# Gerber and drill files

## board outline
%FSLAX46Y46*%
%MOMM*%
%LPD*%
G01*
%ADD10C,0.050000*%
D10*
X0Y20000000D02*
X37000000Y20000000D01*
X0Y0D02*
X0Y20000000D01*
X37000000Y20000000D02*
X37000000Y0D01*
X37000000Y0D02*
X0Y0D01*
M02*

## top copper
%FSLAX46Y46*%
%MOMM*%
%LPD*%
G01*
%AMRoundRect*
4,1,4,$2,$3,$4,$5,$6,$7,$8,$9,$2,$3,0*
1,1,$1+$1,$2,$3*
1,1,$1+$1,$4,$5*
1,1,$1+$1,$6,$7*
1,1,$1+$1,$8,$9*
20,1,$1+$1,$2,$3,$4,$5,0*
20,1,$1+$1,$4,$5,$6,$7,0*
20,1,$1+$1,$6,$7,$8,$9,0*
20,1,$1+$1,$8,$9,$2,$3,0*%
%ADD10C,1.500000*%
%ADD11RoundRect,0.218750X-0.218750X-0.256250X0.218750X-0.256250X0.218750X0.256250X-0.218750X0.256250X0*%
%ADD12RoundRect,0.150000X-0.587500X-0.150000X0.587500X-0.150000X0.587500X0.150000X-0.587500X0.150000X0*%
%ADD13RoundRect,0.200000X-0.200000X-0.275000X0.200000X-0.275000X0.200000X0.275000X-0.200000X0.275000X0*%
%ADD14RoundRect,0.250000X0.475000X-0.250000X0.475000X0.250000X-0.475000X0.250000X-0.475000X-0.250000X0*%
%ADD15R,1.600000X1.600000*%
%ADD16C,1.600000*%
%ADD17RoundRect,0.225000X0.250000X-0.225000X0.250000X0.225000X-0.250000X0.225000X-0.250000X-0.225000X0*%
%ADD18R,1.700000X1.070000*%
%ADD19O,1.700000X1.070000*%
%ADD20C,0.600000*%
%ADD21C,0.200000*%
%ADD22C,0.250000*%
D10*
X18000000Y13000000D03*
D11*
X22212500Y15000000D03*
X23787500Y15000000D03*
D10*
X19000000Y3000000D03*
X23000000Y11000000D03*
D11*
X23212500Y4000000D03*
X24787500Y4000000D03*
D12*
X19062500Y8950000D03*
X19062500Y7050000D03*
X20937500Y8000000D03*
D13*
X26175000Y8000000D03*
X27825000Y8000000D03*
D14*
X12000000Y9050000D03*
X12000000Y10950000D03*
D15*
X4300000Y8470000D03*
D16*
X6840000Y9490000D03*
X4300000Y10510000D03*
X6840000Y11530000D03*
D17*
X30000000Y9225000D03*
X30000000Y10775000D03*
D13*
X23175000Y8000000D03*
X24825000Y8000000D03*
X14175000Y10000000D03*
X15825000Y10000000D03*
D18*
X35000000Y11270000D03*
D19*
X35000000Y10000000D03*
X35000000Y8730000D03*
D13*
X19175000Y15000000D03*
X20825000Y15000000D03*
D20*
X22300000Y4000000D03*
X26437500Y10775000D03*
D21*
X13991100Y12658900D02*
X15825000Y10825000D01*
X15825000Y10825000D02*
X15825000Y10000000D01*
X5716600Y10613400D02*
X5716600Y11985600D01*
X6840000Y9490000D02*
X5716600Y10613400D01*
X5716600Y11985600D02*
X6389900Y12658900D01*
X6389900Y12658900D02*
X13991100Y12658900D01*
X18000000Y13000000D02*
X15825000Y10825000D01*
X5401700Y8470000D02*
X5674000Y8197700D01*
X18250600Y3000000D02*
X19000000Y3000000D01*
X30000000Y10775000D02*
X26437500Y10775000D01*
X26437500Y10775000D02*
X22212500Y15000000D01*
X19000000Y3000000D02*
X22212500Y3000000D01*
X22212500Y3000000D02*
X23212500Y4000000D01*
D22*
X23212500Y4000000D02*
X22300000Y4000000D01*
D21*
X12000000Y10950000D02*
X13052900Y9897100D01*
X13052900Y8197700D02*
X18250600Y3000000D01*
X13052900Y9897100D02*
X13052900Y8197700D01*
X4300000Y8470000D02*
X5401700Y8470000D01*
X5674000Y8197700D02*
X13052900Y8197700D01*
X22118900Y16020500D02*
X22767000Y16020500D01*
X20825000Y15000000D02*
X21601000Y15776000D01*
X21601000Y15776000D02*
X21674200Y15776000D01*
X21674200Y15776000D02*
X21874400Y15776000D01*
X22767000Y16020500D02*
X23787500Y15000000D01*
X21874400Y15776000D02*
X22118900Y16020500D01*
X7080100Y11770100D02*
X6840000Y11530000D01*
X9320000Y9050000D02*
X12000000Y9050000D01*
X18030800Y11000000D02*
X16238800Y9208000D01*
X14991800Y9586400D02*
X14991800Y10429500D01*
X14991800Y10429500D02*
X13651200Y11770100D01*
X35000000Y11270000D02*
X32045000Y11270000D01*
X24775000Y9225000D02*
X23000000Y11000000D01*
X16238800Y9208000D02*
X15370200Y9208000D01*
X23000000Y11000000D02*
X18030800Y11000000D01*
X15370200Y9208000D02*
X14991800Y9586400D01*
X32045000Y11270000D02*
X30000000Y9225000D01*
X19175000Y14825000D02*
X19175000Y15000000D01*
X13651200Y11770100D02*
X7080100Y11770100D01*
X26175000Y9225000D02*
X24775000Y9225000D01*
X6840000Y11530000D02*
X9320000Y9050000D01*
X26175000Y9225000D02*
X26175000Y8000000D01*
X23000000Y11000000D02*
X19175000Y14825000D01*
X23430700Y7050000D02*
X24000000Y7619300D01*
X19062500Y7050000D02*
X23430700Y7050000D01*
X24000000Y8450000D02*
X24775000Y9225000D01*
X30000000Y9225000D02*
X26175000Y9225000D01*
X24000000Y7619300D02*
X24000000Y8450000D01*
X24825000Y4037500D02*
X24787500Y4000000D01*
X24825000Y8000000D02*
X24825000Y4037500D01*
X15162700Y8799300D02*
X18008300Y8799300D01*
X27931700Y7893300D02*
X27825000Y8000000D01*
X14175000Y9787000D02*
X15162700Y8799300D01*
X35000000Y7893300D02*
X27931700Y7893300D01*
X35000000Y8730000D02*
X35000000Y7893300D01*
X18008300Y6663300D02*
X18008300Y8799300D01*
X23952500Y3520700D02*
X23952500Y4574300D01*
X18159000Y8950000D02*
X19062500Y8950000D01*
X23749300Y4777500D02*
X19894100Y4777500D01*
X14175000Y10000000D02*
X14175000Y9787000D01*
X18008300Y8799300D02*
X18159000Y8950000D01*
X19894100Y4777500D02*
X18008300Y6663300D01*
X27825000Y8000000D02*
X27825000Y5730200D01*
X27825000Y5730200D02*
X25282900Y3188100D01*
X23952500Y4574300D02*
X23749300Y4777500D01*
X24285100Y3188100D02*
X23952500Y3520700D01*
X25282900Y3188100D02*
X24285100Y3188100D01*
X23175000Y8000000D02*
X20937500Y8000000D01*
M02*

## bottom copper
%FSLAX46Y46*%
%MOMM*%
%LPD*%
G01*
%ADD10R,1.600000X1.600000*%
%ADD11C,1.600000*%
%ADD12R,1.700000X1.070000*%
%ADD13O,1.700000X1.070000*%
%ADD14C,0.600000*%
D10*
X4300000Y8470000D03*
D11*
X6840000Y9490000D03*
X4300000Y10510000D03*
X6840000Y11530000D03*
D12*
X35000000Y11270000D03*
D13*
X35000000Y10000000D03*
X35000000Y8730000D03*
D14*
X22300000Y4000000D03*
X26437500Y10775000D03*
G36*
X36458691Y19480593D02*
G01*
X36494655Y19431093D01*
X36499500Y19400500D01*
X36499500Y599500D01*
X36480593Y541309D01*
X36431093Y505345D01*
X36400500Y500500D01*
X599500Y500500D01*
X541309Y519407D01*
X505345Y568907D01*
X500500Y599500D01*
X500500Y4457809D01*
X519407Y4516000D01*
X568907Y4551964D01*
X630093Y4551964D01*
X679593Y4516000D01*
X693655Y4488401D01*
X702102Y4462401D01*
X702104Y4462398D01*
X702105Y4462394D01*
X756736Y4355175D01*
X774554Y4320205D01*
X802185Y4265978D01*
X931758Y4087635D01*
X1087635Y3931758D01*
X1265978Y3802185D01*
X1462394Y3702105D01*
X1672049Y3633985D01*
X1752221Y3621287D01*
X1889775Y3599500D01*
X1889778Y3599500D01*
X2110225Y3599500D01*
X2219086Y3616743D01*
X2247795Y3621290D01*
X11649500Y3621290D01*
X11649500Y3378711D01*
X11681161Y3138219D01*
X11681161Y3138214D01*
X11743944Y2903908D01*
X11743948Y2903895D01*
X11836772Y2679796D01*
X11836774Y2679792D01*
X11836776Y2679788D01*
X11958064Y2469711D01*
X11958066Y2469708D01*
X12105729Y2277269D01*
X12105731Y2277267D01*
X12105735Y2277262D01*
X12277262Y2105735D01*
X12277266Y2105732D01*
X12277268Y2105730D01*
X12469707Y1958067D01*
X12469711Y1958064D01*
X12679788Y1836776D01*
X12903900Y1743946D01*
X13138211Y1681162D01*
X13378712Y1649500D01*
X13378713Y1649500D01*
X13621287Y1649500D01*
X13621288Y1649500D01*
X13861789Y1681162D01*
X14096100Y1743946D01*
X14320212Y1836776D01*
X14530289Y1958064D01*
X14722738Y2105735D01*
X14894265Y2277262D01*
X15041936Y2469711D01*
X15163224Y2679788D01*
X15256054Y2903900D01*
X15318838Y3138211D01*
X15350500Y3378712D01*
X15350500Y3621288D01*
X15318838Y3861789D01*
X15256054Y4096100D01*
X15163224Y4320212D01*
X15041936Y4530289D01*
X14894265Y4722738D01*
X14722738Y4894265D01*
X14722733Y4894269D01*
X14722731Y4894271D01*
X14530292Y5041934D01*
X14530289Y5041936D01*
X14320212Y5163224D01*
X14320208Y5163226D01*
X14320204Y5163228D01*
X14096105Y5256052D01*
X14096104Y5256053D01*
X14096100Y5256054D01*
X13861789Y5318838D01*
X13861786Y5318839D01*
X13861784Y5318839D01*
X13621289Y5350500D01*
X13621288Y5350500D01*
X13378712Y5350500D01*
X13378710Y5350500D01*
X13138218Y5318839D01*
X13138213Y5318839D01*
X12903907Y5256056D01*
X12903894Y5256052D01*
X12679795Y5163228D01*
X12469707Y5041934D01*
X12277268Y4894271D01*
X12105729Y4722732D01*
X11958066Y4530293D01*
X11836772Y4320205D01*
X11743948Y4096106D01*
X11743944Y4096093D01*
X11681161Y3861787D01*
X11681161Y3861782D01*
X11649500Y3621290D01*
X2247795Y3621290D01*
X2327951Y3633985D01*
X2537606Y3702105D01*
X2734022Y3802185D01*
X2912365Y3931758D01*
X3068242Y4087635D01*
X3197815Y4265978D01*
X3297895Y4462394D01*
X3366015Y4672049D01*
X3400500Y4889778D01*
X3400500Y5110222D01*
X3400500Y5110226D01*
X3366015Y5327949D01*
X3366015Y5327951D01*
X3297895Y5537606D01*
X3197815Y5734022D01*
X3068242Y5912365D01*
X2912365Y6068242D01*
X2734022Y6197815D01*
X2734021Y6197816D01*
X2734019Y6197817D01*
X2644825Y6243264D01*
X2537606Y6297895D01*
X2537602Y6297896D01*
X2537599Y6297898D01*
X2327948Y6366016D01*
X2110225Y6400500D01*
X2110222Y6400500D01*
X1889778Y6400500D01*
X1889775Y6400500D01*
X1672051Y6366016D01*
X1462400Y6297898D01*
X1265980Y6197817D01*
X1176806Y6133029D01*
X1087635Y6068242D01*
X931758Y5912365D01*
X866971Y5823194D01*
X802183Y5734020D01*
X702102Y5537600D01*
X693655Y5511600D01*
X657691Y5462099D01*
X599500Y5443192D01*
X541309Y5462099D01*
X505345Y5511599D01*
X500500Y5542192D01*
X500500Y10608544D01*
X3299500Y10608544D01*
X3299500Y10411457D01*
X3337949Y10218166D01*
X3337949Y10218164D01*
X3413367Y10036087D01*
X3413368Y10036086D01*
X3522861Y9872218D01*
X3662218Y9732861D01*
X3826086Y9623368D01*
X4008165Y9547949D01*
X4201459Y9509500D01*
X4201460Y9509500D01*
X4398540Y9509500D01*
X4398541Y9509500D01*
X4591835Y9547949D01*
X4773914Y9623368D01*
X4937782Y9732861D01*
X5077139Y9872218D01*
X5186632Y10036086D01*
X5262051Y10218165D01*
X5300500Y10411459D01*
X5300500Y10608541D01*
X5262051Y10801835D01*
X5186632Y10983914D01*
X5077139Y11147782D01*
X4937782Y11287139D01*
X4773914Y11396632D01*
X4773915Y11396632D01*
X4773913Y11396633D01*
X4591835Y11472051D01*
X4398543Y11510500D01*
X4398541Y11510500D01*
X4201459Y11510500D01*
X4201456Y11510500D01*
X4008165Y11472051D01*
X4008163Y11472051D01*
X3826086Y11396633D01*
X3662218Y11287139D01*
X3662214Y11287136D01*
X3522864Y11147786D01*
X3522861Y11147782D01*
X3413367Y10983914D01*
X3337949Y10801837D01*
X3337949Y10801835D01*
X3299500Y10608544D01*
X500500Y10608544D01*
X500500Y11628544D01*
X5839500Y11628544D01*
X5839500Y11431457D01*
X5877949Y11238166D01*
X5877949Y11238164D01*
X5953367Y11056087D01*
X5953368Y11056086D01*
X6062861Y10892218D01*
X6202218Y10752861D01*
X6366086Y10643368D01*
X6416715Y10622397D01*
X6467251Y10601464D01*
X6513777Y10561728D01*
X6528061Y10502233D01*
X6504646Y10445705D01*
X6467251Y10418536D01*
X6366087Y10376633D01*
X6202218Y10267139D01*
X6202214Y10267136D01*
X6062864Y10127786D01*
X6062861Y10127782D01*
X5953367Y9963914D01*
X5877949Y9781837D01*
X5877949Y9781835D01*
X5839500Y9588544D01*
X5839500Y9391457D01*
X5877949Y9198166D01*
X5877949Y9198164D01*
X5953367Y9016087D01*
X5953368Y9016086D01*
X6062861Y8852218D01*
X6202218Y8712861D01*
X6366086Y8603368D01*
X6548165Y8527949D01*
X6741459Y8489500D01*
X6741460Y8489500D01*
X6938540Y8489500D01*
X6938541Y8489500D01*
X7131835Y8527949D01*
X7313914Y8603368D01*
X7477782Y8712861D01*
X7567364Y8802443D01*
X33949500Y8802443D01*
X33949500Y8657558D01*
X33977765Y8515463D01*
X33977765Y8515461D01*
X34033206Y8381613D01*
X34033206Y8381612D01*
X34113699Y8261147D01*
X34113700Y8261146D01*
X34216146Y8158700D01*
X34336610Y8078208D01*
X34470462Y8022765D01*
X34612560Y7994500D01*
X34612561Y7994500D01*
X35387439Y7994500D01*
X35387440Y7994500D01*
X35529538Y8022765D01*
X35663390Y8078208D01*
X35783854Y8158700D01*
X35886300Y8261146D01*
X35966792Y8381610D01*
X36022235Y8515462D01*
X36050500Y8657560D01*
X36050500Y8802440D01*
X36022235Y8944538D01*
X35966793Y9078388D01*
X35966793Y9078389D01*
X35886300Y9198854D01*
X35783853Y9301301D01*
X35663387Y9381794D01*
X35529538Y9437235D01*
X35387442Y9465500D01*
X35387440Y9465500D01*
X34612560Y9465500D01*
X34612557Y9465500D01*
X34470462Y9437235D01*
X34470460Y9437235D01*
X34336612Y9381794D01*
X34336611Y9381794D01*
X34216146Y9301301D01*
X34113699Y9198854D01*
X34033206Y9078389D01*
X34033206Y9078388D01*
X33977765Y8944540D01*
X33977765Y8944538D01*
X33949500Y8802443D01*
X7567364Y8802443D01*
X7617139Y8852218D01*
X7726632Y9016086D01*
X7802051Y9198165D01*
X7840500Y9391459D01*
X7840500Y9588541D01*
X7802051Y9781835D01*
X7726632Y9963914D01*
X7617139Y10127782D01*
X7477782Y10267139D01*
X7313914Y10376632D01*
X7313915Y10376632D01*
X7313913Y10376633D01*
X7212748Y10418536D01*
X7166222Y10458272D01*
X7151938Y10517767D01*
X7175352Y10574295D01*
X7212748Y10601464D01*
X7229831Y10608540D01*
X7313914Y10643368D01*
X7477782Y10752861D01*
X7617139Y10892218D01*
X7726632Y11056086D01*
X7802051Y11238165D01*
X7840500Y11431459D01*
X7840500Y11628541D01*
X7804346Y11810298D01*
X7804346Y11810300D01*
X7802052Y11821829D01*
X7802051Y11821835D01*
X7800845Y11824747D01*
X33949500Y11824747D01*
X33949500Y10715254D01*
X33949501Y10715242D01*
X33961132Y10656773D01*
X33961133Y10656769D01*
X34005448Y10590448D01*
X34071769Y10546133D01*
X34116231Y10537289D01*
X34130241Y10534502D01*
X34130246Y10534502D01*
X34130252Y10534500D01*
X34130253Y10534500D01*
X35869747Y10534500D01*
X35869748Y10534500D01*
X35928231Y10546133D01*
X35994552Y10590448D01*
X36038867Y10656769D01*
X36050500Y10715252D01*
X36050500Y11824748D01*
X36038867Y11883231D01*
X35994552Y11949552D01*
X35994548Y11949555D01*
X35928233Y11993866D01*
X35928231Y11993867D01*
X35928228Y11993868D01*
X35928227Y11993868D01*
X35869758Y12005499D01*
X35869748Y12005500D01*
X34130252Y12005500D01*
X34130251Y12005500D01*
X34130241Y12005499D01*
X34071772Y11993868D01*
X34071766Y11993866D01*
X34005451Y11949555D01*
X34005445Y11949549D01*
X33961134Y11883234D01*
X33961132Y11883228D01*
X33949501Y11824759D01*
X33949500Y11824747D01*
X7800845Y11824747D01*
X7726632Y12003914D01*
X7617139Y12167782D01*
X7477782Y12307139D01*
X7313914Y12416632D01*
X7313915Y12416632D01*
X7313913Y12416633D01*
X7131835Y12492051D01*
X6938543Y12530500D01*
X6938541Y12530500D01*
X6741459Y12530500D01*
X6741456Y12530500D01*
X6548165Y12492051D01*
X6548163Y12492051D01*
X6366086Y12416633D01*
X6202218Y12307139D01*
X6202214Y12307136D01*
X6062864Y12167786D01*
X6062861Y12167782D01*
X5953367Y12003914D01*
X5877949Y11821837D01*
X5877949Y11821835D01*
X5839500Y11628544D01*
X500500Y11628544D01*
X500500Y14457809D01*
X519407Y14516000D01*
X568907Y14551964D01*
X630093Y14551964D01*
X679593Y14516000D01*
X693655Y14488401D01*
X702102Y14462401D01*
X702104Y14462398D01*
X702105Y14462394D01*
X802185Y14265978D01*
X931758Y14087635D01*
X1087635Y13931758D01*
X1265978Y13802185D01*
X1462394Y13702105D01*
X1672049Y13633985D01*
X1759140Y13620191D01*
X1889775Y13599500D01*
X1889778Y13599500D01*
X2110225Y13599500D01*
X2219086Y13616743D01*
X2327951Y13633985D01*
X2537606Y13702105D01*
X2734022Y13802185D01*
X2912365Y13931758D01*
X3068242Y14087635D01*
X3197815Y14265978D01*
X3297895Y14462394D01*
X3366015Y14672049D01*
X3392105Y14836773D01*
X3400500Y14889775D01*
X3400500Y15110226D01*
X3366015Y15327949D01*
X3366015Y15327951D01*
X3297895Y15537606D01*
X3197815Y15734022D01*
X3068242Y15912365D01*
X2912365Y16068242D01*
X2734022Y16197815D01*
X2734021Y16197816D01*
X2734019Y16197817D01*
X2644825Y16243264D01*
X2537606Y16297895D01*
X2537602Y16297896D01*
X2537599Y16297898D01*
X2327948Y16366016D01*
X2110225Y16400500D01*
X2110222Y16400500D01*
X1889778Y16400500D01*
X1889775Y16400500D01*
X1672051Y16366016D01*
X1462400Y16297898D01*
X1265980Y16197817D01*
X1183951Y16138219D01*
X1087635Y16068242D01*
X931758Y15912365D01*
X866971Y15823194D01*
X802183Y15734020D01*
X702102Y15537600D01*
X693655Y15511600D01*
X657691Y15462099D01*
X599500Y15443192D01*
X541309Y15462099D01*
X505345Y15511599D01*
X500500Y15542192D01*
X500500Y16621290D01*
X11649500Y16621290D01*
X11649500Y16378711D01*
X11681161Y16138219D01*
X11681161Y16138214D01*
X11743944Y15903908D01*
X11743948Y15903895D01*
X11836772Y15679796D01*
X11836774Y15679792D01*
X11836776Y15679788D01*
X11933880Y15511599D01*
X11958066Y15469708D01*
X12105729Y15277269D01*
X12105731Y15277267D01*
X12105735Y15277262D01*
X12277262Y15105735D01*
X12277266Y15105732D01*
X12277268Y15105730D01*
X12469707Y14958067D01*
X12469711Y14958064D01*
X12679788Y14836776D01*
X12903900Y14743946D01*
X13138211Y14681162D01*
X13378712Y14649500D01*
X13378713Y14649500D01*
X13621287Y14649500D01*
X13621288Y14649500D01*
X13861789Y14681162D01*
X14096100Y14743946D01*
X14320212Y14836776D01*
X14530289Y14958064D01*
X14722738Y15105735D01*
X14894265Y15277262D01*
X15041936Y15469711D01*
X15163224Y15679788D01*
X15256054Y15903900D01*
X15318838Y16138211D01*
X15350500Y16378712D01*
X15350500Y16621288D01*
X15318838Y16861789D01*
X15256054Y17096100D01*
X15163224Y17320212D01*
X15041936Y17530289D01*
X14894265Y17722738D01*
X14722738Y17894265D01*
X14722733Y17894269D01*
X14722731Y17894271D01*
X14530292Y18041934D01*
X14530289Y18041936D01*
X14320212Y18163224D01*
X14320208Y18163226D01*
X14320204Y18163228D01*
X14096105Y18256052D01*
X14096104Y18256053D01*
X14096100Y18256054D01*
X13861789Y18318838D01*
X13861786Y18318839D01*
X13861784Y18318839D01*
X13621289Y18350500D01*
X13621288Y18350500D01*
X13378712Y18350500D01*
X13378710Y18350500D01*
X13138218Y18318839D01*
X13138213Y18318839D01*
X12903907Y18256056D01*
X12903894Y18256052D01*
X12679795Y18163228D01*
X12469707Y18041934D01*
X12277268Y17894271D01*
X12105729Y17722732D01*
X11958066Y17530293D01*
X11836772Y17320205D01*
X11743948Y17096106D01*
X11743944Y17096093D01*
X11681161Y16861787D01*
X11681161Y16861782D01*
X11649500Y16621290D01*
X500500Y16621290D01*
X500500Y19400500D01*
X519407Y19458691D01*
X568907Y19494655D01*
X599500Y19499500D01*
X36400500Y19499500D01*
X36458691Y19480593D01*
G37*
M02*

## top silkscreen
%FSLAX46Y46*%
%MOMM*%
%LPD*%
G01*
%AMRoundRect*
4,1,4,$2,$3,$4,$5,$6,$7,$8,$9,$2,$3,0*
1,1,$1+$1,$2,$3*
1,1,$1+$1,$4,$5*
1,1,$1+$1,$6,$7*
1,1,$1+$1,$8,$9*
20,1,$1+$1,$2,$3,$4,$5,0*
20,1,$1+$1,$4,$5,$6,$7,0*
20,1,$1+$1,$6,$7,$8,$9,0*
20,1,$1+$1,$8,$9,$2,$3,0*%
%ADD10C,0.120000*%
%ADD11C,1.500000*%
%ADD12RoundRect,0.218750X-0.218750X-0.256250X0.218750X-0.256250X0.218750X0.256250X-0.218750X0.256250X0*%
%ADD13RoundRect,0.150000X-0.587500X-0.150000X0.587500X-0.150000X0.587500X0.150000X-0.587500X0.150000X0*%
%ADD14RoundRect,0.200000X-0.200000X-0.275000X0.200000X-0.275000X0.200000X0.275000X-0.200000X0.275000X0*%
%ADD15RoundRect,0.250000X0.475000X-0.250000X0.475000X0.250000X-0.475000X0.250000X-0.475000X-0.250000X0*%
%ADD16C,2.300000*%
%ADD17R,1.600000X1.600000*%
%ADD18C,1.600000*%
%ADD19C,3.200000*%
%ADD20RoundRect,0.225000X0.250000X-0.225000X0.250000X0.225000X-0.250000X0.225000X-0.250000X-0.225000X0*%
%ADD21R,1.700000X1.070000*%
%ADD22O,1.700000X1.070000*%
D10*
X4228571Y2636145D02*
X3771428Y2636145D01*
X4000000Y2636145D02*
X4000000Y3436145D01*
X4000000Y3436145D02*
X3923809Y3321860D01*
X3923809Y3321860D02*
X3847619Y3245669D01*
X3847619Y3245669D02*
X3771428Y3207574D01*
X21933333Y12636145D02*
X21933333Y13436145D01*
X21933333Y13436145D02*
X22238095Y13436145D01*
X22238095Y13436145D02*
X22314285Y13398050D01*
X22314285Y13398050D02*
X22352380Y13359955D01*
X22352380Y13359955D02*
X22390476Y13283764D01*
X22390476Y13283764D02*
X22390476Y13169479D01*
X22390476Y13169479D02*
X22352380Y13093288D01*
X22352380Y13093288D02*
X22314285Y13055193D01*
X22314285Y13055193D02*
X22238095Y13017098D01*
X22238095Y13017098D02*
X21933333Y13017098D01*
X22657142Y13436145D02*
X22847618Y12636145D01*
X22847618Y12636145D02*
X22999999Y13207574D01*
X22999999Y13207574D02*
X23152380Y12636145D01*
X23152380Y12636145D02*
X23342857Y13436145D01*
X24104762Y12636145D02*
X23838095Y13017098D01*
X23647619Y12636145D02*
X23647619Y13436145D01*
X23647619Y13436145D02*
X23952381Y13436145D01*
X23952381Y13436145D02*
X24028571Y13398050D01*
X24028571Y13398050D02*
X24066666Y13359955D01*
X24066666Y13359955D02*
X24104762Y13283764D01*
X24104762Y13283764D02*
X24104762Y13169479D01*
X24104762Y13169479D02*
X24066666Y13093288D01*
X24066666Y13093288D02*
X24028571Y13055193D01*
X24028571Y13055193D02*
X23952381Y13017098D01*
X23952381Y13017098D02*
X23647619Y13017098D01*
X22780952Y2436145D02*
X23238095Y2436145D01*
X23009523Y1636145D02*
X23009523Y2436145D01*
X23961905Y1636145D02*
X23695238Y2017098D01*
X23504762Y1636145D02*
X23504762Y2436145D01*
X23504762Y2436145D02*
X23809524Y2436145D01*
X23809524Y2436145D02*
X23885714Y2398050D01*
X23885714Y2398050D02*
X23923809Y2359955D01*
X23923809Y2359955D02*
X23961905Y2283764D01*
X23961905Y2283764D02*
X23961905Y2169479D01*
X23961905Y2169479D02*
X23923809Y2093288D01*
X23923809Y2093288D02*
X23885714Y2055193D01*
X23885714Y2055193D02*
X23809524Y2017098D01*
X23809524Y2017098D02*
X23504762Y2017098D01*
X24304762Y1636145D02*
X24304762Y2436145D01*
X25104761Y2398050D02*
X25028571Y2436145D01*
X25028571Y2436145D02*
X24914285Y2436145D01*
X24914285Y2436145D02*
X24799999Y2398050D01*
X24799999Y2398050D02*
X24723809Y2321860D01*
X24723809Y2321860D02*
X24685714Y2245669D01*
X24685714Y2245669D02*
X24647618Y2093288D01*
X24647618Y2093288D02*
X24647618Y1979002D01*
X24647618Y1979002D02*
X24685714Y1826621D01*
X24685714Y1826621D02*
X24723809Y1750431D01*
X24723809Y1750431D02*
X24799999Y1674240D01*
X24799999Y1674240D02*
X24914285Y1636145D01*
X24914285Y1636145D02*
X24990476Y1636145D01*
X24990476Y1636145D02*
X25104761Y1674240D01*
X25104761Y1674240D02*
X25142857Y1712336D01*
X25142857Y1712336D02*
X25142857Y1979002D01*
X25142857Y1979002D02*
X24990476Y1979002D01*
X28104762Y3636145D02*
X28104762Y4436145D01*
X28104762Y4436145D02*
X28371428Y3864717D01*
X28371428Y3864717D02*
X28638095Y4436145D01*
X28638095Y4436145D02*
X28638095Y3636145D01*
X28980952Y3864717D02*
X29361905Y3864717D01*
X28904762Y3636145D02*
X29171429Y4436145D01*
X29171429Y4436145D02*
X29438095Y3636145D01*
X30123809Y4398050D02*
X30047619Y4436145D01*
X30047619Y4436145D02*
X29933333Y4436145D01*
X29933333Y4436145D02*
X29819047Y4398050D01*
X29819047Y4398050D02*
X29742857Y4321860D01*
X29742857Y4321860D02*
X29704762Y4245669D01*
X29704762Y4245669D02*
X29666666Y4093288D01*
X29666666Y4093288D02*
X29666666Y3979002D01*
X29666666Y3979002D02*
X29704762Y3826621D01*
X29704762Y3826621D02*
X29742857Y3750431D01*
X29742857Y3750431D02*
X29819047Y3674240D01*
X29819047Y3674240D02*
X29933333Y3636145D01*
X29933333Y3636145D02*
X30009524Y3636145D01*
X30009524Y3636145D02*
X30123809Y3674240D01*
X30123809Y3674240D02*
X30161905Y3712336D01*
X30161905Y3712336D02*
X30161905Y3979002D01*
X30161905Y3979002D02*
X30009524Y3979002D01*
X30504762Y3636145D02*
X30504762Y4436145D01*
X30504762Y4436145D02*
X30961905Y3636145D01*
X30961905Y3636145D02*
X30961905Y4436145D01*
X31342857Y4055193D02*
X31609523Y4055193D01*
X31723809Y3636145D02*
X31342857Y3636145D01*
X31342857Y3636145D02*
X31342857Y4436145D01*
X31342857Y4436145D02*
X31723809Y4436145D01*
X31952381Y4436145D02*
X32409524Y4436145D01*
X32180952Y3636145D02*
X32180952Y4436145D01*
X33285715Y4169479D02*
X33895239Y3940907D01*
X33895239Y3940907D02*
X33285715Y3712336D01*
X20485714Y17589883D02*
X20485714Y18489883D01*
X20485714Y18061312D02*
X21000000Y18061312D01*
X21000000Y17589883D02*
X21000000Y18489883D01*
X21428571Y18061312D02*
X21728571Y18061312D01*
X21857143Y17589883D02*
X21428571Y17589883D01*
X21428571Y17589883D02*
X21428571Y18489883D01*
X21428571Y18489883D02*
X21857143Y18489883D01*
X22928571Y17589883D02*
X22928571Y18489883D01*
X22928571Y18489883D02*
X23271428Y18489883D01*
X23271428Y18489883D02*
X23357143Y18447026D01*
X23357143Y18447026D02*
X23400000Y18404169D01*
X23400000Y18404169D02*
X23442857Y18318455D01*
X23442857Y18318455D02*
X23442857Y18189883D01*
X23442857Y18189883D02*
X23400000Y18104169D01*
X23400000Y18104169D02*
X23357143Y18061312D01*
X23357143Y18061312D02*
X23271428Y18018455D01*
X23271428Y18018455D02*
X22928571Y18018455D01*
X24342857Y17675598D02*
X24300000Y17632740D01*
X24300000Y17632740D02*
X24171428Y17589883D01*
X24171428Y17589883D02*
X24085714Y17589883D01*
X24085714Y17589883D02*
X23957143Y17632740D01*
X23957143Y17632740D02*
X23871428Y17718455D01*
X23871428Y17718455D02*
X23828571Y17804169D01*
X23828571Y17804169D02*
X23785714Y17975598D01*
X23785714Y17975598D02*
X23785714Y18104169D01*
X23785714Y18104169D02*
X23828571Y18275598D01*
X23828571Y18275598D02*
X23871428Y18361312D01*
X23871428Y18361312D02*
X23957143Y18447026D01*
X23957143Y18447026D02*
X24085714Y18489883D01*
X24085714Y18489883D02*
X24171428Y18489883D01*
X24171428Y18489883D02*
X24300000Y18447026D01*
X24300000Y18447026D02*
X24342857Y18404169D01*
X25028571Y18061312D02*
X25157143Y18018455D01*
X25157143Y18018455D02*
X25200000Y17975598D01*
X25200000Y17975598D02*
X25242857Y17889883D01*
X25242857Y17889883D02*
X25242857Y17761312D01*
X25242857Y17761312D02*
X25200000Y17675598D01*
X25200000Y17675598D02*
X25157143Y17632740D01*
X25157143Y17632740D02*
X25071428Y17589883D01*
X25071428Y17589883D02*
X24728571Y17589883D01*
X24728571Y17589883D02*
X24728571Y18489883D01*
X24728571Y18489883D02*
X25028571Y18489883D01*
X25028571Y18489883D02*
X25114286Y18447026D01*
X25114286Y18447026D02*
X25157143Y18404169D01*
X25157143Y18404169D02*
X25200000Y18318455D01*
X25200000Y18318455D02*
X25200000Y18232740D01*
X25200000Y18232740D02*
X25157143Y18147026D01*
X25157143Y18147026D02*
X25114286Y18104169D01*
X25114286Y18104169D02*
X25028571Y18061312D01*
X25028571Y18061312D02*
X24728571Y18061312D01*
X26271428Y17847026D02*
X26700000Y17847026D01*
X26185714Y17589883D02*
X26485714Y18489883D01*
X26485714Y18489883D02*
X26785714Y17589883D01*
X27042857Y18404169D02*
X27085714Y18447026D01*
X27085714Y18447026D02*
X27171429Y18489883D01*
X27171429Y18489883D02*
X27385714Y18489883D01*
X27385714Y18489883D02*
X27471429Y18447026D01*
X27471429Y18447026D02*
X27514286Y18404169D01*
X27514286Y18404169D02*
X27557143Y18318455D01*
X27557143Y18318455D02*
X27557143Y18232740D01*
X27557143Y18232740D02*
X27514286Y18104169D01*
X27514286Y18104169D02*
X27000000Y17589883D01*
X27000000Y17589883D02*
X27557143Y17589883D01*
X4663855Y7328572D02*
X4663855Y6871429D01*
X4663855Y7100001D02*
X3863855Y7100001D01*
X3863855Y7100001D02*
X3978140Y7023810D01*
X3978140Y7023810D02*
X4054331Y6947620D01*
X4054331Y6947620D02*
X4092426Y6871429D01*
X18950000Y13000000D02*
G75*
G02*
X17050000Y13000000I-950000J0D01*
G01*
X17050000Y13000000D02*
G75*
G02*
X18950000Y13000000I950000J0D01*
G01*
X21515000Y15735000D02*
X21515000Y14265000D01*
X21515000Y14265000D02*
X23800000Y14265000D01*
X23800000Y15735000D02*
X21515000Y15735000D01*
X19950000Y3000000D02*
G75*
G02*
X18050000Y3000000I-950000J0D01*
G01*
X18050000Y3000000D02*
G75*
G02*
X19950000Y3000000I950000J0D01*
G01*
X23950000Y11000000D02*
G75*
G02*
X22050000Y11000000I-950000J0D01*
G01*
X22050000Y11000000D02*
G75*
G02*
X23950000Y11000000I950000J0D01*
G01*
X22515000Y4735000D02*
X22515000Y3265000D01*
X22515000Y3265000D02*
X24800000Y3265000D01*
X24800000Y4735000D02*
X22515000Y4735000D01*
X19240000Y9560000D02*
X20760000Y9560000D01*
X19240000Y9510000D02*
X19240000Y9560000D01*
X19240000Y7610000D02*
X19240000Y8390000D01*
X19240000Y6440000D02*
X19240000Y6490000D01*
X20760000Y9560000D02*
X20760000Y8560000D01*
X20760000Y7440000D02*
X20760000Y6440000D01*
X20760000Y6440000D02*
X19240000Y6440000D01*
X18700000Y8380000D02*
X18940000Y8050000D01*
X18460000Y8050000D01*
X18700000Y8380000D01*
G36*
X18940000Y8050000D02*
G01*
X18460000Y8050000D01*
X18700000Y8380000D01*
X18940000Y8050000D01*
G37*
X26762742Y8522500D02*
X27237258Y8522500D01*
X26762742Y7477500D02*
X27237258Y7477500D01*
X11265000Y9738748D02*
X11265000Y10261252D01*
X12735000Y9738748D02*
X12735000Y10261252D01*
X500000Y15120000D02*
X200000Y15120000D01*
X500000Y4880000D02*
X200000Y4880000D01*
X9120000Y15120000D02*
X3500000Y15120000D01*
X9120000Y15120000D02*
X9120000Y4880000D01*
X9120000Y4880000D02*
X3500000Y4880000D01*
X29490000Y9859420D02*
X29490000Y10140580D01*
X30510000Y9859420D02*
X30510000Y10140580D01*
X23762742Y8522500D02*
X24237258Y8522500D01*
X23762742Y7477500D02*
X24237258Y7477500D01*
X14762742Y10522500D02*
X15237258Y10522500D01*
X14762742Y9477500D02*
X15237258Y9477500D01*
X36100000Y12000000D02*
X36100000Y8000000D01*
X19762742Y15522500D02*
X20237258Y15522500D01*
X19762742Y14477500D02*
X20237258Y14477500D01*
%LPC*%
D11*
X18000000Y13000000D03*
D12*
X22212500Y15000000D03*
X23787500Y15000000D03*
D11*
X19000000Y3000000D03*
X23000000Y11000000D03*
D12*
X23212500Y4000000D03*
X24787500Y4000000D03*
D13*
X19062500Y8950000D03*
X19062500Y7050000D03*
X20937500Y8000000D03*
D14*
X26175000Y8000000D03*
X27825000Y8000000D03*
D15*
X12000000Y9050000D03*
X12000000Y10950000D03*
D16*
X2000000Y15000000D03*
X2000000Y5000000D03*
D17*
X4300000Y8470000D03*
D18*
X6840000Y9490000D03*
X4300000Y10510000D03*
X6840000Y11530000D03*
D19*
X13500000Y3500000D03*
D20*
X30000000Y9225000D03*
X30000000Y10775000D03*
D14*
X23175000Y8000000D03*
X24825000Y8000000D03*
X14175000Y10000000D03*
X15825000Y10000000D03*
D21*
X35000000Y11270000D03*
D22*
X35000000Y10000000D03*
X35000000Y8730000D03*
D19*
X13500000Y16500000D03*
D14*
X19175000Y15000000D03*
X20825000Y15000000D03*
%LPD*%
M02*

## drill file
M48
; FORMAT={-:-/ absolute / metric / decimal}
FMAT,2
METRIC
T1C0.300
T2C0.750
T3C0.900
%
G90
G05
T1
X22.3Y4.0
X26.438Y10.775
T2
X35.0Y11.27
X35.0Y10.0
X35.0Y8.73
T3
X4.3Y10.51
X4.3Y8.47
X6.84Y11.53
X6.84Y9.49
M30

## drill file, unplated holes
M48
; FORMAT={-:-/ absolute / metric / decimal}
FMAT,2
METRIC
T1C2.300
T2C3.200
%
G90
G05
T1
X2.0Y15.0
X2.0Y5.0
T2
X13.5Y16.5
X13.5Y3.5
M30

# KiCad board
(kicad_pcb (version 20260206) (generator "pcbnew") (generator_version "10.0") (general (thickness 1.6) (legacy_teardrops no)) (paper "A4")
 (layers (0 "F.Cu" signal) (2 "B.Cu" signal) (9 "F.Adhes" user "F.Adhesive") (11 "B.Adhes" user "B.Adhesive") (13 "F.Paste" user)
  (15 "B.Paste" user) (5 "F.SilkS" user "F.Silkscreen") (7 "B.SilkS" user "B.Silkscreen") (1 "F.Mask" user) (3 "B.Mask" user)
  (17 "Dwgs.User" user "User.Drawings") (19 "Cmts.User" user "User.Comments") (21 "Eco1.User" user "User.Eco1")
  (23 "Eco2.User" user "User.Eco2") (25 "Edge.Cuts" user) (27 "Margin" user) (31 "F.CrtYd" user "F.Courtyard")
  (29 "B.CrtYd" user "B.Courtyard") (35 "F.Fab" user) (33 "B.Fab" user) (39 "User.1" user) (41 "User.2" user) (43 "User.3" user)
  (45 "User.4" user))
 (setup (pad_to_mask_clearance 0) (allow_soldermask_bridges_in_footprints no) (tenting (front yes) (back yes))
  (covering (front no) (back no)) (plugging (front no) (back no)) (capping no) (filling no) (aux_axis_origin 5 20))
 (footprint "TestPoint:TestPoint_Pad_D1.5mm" (layer "F.Cu") (at 23 7)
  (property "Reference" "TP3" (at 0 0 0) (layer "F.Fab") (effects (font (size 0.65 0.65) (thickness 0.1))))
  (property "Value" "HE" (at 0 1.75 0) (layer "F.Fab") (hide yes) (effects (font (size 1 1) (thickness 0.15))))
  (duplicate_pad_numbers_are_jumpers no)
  (fp_circle (center 0 0) (end 0 0.95) (stroke (width 0.12) (type solid)) (fill no) (layer "F.SilkS"))
  (pad "1" smd circle (at 0 0) (size 1.5 1.5) (layers "F.Cu" "F.Mask") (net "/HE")))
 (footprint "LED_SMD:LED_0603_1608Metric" (layer "F.Cu") (at 28 5)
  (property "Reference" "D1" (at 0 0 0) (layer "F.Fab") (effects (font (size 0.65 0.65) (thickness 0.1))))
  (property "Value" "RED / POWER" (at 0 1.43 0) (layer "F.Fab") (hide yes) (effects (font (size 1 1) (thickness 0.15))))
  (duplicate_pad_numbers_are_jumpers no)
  (fp_line (start -1.485 -0.735) (end -1.485 0.735) (stroke (width 0.12) (type solid)) (layer "F.SilkS"))
  (fp_line (start -1.485 0.735) (end 0.8 0.735) (stroke (width 0.12) (type solid)) (layer "F.SilkS"))
  (fp_line (start 0.8 -0.735) (end -1.485 -0.735) (stroke (width 0.12) (type solid)) (layer "F.SilkS"))
  (pad "1" smd roundrect (at -0.7875 0) (size 0.875 0.95) (layers "F.Cu" "F.Mask" "F.Paste") (roundrect_rratio 0.25) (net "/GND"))
  (pad "2" smd roundrect (at 0.7875 0) (size 0.875 0.95) (layers "F.Cu" "F.Mask" "F.Paste") (roundrect_rratio 0.25) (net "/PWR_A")))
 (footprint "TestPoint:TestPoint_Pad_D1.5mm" (layer "F.Cu") (at 24 17)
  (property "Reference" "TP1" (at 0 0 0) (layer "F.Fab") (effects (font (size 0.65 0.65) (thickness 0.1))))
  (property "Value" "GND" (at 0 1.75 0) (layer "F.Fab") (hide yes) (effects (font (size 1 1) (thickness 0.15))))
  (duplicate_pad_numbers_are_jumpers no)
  (fp_circle (center 0 0) (end 0 0.95) (stroke (width 0.12) (type solid)) (fill no) (layer "F.SilkS"))
  (pad "1" smd circle (at 0 0) (size 1.5 1.5) (layers "F.Cu" "F.Mask") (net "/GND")))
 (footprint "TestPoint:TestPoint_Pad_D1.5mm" (layer "F.Cu") (at 28 9)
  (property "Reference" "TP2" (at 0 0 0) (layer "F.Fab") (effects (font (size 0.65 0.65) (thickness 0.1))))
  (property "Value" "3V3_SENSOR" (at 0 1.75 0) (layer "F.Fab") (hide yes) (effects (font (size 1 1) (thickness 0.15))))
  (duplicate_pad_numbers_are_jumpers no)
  (fp_circle (center 0 0) (end 0 0.95) (stroke (width 0.12) (type solid)) (fill no) (layer "F.SilkS"))
  (pad "1" smd circle (at 0 0) (size 1.5 1.5) (layers "F.Cu" "F.Mask") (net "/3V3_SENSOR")))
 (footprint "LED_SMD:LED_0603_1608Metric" (layer "F.Cu") (at 29 16)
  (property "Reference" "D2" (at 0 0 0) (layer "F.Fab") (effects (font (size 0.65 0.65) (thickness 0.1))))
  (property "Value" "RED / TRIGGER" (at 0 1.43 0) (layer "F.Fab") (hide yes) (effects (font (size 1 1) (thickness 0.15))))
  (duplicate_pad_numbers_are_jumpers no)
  (fp_line (start -1.485 -0.735) (end -1.485 0.735) (stroke (width 0.12) (type solid)) (layer "F.SilkS"))
  (fp_line (start -1.485 0.735) (end 0.8 0.735) (stroke (width 0.12) (type solid)) (layer "F.SilkS"))
  (fp_line (start 0.8 -0.735) (end -1.485 -0.735) (stroke (width 0.12) (type solid)) (layer "F.SilkS"))
  (pad "1" smd roundrect (at -0.7875 0) (size 0.875 0.95) (layers "F.Cu" "F.Mask" "F.Paste") (roundrect_rratio 0.25) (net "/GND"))
  (pad "2" smd roundrect (at 0.7875 0) (size 0.875 0.95) (layers "F.Cu" "F.Mask" "F.Paste") (roundrect_rratio 0.25) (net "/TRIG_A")))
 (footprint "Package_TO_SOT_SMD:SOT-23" (layer "F.Cu") (at 25 12)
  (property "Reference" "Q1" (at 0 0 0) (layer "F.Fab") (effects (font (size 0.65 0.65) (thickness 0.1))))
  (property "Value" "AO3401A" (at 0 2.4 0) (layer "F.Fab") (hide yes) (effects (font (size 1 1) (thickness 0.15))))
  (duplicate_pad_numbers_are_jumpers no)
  (fp_line (start -0.76 -1.56) (end 0.76 -1.56) (stroke (width 0.12) (type solid)) (layer "F.SilkS"))
  (fp_line (start -0.76 -1.51) (end -0.76 -1.56) (stroke (width 0.12) (type solid)) (layer "F.SilkS"))
  (fp_line (start -0.76 0.39) (end -0.76 -0.39) (stroke (width 0.12) (type solid)) (layer "F.SilkS"))
  (fp_line (start -0.76 1.56) (end -0.76 1.51) (stroke (width 0.12) (type solid)) (layer "F.SilkS"))
  (fp_line (start 0.76 -1.56) (end 0.76 -0.56) (stroke (width 0.12) (type solid)) (layer "F.SilkS"))
  (fp_line (start 0.76 0.56) (end 0.76 1.56) (stroke (width 0.12) (type solid)) (layer "F.SilkS"))
  (fp_line (start 0.76 1.56) (end -0.76 1.56) (stroke (width 0.12) (type solid)) (layer "F.SilkS"))
  (fp_poly (pts (xy -1.3 -0.38) (xy -1.06 -0.05) (xy -1.54 -0.05)) (stroke (width 0.12) (type solid)) (fill yes) (layer "F.SilkS"))
  (pad "1" smd roundrect (at -0.9375 -0.95) (size 1.475 0.6) (layers "F.Cu" "F.Mask" "F.Paste") (roundrect_rratio 0.25) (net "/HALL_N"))
  (pad "2" smd roundrect (at -0.9375 0.95) (size 1.475 0.6) (layers "F.Cu" "F.Mask" "F.Paste") (roundrect_rratio 0.25) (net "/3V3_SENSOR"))
  (pad "3" smd roundrect (at 0.9375 0) (size 1.475 0.6) (layers "F.Cu" "F.Mask" "F.Paste") (roundrect_rratio 0.25) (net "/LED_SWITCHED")))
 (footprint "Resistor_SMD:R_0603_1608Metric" (layer "F.Cu") (at 32 12)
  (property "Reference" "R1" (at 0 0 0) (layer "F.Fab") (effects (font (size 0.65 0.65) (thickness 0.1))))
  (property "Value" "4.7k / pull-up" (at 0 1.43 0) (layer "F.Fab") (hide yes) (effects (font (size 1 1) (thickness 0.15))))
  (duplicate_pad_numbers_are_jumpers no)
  (fp_line (start -0.237258 -0.5225) (end 0.237258 -0.5225) (stroke (width 0.12) (type solid)) (layer "F.SilkS"))
  (fp_line (start -0.237258 0.5225) (end 0.237258 0.5225) (stroke (width 0.12) (type solid)) (layer "F.SilkS"))
  (pad "1" smd roundrect (at -0.825 0) (size 0.8 0.95) (layers "F.Cu" "F.Mask" "F.Paste") (roundrect_rratio 0.25) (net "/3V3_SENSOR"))
  (pad "2" smd roundrect (at 0.825 0) (size 0.8 0.95) (layers "F.Cu" "F.Mask" "F.Paste") (roundrect_rratio 0.25) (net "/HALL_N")))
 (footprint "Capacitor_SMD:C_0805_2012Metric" (layer "F.Cu") (at 17 10 90)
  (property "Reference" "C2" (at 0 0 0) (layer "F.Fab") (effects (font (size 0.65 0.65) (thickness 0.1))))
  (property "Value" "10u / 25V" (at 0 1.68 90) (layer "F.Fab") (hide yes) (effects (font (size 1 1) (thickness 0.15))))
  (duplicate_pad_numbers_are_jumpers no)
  (fp_line (start -0.261252 -0.735) (end 0.261252 -0.735) (stroke (width 0.12) (type solid)) (layer "F.SilkS"))
  (fp_line (start -0.261252 0.735) (end 0.261252 0.735) (stroke (width 0.12) (type solid)) (layer "F.SilkS"))
  (pad "1" smd roundrect (at -0.95 0 90) (size 1 1.45) (layers "F.Cu" "F.Mask" "F.Paste") (roundrect_rratio 0.25) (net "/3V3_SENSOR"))
  (pad "2" smd roundrect (at 0.95 0 90) (size 1 1.45) (layers "F.Cu" "F.Mask" "F.Paste") (roundrect_rratio 0.25) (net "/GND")))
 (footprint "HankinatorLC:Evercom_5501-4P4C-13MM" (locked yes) (layer "F.Cu") (at 7 10 -90)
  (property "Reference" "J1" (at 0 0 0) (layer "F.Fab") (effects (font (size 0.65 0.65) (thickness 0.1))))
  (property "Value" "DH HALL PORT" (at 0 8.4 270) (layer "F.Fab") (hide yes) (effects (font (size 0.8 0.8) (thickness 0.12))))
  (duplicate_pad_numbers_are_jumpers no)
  (fp_line (start -5.12 1.5) (end -5.12 1.8) (stroke (width 0.12) (type default)) (layer "F.SilkS"))
  (fp_line (start 5.12 1.5) (end 5.12 1.8) (stroke (width 0.12) (type default)) (layer "F.SilkS"))
  (fp_line (start -5.12 -7.12) (end -5.12 -1.5) (stroke (width 0.12) (type default)) (layer "F.SilkS"))
  (fp_line (start -5.12 -7.12) (end 5.12 -7.12) (stroke (width 0.12) (type default)) (layer "F.SilkS"))
  (fp_line (start 5.12 -7.12) (end 5.12 -1.5) (stroke (width 0.12) (type default)) (layer "F.SilkS"))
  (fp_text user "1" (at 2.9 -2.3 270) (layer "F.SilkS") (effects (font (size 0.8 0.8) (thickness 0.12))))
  (pad "" np_thru_hole circle (at -5 0 270) (size 2.3 2.3) (drill 2.3) (layers "*.Cu" "*.Mask"))
  (pad "" np_thru_hole circle (at 5 0 270) (size 2.3 2.3) (drill 2.3) (layers "*.Cu" "*.Mask"))
  (pad "1" thru_hole rect (at 1.53 -2.3 270) (size 1.6 1.6) (drill 0.9) (layers "*.Cu" "*.Mask") (remove_unused_layers no) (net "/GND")
   (zone_connect 2))
  (pad "2" thru_hole circle (at 0.51 -4.84 270) (size 1.6 1.6) (drill 0.9) (layers "*.Cu" "*.Mask") (remove_unused_layers no) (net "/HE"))
  (pad "3" thru_hole circle (at -0.51 -2.3 270) (size 1.6 1.6) (drill 0.9) (layers "*.Cu" "*.Mask") (remove_unused_layers no)
   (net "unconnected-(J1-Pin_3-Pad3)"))
  (pad "4" thru_hole circle (at -1.53 -4.84 270) (size 1.6 1.6) (drill 0.9) (layers "*.Cu" "*.Mask") (remove_unused_layers no)
   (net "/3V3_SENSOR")))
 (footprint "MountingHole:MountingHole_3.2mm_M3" (layer "F.Cu") (at 18.5 16.5)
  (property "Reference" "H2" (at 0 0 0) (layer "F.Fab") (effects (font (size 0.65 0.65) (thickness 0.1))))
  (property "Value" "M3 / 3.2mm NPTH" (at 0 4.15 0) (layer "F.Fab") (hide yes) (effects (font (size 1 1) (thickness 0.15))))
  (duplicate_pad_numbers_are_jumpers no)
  (pad "" np_thru_hole circle (at 0 0) (size 3.2 3.2) (drill 3.2) (layers "*.Cu" "*.Mask")))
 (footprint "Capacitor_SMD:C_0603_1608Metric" (layer "F.Cu") (at 35 10 90)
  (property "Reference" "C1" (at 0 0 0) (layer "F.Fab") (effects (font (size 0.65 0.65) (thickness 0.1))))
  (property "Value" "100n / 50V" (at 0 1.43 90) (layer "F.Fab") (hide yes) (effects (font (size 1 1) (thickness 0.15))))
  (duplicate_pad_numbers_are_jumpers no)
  (fp_line (start -0.14058 -0.51) (end 0.14058 -0.51) (stroke (width 0.12) (type solid)) (layer "F.SilkS"))
  (fp_line (start -0.14058 0.51) (end 0.14058 0.51) (stroke (width 0.12) (type solid)) (layer "F.SilkS"))
  (pad "1" smd roundrect (at -0.775 0 90) (size 0.9 0.95) (layers "F.Cu" "F.Mask" "F.Paste") (roundrect_rratio 0.25) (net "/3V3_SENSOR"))
  (pad "2" smd roundrect (at 0.775 0 90) (size 0.9 0.95) (layers "F.Cu" "F.Mask" "F.Paste") (roundrect_rratio 0.25) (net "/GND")))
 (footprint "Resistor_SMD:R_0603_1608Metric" (layer "F.Cu") (at 29 12)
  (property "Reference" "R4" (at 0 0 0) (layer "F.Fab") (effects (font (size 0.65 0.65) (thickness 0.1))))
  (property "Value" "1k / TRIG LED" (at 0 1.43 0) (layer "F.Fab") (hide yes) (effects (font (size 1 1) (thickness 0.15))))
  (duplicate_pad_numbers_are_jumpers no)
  (fp_line (start -0.237258 -0.5225) (end 0.237258 -0.5225) (stroke (width 0.12) (type solid)) (layer "F.SilkS"))
  (fp_line (start -0.237258 0.5225) (end 0.237258 0.5225) (stroke (width 0.12) (type solid)) (layer "F.SilkS"))
  (pad "1" smd roundrect (at -0.825 0) (size 0.8 0.95) (layers "F.Cu" "F.Mask" "F.Paste") (roundrect_rratio 0.25) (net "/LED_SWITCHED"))
  (pad "2" smd roundrect (at 0.825 0) (size 0.8 0.95) (layers "F.Cu" "F.Mask" "F.Paste") (roundrect_rratio 0.25) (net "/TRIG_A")))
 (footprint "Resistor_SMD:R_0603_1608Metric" (layer "F.Cu") (at 20 10)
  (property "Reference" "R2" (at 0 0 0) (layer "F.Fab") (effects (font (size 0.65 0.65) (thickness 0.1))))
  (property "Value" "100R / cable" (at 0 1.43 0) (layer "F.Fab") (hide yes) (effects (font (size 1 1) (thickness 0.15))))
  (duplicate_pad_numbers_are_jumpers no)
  (fp_line (start -0.237258 -0.5225) (end 0.237258 -0.5225) (stroke (width 0.12) (type solid)) (layer "F.SilkS"))
  (fp_line (start -0.237258 0.5225) (end 0.237258 0.5225) (stroke (width 0.12) (type solid)) (layer "F.SilkS"))
  (pad "1" smd roundrect (at -0.825 0) (size 0.8 0.95) (layers "F.Cu" "F.Mask" "F.Paste") (roundrect_rratio 0.25) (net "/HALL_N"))
  (pad "2" smd roundrect (at 0.825 0) (size 0.8 0.95) (layers "F.Cu" "F.Mask" "F.Paste") (roundrect_rratio 0.25) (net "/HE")))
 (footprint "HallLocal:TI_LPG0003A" (layer "F.Cu") (at 40 8.73 -90)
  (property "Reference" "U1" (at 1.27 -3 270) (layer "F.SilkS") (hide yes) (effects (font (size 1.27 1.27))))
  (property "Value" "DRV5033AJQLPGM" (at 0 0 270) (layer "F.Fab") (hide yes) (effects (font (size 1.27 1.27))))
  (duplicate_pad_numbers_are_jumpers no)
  (fp_line (start -0.73 -1.1) (end 3.27 -1.1) (stroke (width 0.12) (type default)) (layer "F.SilkS"))
  (pad "1" thru_hole rect (at 0 0 270) (size 1.07 1.7) (drill 0.75) (layers "*.Cu" "*.Mask") (remove_unused_layers no) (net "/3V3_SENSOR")
   (thermal_bridge_angle 45))
  (pad "2" thru_hole oval (at 1.27 0 270) (size 1.07 1.7) (drill 0.75) (layers "*.Cu" "*.Mask") (remove_unused_layers no) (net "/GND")
   (zone_connect 2) (thermal_bridge_angle 45))
  (pad "3" thru_hole oval (at 2.54 0 270) (size 1.07 1.7) (drill 0.75) (layers "*.Cu" "*.Mask") (remove_unused_layers no) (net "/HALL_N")
   (thermal_bridge_angle 45)))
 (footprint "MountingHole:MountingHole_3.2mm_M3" (layer "F.Cu") (at 18.5 3.5)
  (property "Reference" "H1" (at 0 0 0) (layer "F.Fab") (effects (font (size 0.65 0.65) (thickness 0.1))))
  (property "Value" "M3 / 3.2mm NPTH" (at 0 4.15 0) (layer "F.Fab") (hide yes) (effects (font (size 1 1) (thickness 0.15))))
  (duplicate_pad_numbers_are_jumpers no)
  (pad "" np_thru_hole circle (at 0 0) (size 3.2 3.2) (drill 3.2) (layers "*.Cu" "*.Mask")))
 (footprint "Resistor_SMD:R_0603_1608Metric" (layer "F.Cu") (at 25 5)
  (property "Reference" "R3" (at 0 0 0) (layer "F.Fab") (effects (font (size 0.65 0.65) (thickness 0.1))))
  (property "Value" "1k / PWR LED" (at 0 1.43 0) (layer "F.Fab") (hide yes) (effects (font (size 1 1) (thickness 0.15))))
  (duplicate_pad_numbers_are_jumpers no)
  (fp_line (start -0.237258 -0.5225) (end 0.237258 -0.5225) (stroke (width 0.12) (type solid)) (layer "F.SilkS"))
  (fp_line (start -0.237258 0.5225) (end 0.237258 0.5225) (stroke (width 0.12) (type solid)) (layer "F.SilkS"))
  (pad "1" smd roundrect (at -0.825 0) (size 0.8 0.95) (layers "F.Cu" "F.Mask" "F.Paste") (roundrect_rratio 0.25) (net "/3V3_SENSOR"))
  (pad "2" smd roundrect (at 0.825 0) (size 0.8 0.95) (layers "F.Cu" "F.Mask" "F.Paste") (roundrect_rratio 0.25) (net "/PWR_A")))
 (gr_line (start 5 0) (end 42 0) (stroke (width 0.05) (type default)) (layer "Edge.Cuts"))
 (gr_line (start 5 20) (end 5 0) (stroke (width 0.05) (type default)) (layer "Edge.Cuts"))
 (gr_line (start 42 0) (end 42 20) (stroke (width 0.05) (type default)) (layer "Edge.Cuts"))
 (gr_line (start 42 20) (end 5 20) (stroke (width 0.05) (type default)) (layer "Edge.Cuts"))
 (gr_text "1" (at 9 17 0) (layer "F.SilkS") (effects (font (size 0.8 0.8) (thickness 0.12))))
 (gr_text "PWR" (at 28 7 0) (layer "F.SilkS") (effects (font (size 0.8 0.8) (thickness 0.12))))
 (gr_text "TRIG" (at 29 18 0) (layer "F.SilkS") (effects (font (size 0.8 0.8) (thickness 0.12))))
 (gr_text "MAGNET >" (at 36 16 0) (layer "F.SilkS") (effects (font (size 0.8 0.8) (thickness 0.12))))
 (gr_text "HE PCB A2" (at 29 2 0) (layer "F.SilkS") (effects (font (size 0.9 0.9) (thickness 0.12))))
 (segment (start 18.9911 7.3411) (end 20.825 9.175) (width 0.2) (layer "F.Cu") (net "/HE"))
 (segment (start 20.825 9.175) (end 20.825 10) (width 0.2) (layer "F.Cu") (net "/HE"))
 (segment (start 10.7166 9.3866) (end 10.7166 8.0144) (width 0.2) (layer "F.Cu") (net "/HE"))
 (segment (start 11.84 10.51) (end 10.7166 9.3866) (width 0.2) (layer "F.Cu") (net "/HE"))
 (segment (start 10.7166 8.0144) (end 11.3899 7.3411) (width 0.2) (layer "F.Cu") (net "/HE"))
 (segment (start 11.3899 7.3411) (end 18.9911 7.3411) (width 0.2) (layer "F.Cu") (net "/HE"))
 (segment (start 23 7) (end 20.825 9.175) (width 0.2) (layer "F.Cu") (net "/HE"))
 (segment (start 10.4017 11.53) (end 10.674 11.8023) (width 0.2) (layer "F.Cu") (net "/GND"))
 (segment (start 23.2506 17) (end 24 17) (width 0.2) (layer "F.Cu") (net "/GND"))
 (segment (start 35 9.225) (end 31.4375 9.225) (width 0.2) (layer "F.Cu") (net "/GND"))
 (segment (start 31.4375 9.225) (end 27.2125 5) (width 0.2) (layer "F.Cu") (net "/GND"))
 (segment (start 24 17) (end 27.2125 17) (width 0.2) (layer "F.Cu") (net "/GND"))
 (segment (start 27.2125 17) (end 28.2125 16) (width 0.2) (layer "F.Cu") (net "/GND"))
 (segment (start 28.2125 16) (end 27.3 16) (width 0.25) (layer "F.Cu") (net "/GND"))
 (segment (start 17 9.05) (end 18.0529 10.1029) (width 0.2) (layer "F.Cu") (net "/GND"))
 (segment (start 18.0529 11.8023) (end 23.2506 17) (width 0.2) (layer "F.Cu") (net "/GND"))
 (segment (start 18.0529 10.1029) (end 18.0529 11.8023) (width 0.2) (layer "F.Cu") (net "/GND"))
 (segment (start 9.3 11.53) (end 10.4017 11.53) (width 0.2) (layer "F.Cu") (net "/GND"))
 (segment (start 10.674 11.8023) (end 18.0529 11.8023) (width 0.2) (layer "F.Cu") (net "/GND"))
 (via (at 27.3 16) (size 0.6) (drill 0.3) (layers "F.Cu" "B.Cu") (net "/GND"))
 (via (at 31.4375 9.225) (size 0.6) (drill 0.3) (layers "F.Cu" "B.Cu") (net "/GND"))
 (segment (start 27.1189 3.9795) (end 27.767 3.9795) (width 0.2) (layer "F.Cu") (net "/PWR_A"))
 (segment (start 25.825 5) (end 26.601 4.224) (width 0.2) (layer "F.Cu") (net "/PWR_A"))
 (segment (start 26.601 4.224) (end 26.6742 4.224) (width 0.2) (layer "F.Cu") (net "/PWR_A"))
 (segment (start 26.6742 4.224) (end 26.8744 4.224) (width 0.2) (layer "F.Cu") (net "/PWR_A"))
 (segment (start 27.767 3.9795) (end 28.7875 5) (width 0.2) (layer "F.Cu") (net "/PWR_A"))
 (segment (start 26.8744 4.224) (end 27.1189 3.9795) (width 0.2) (layer "F.Cu") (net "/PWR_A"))
 (segment (start 12.0801 8.2299) (end 11.84 8.47) (width 0.2) (layer "F.Cu") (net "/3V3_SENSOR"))
 (segment (start 14.32 10.95) (end 17 10.95) (width 0.2) (layer "F.Cu") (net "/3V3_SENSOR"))
 (segment (start 23.0308 9) (end 21.2388 10.792) (width 0.2) (layer "F.Cu") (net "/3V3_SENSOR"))
 (segment (start 19.9918 10.4136) (end 19.9918 9.5705) (width 0.2) (layer "F.Cu") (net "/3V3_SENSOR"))
 (segment (start 19.9918 9.5705) (end 18.6512 8.2299) (width 0.2) (layer "F.Cu") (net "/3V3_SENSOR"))
 (segment (start 40 8.73) (end 37.045 8.73) (width 0.2) (layer "F.Cu") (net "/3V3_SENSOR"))
 (segment (start 29.775 10.775) (end 28 9) (width 0.2) (layer "F.Cu") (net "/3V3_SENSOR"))
 (segment (start 21.2388 10.792) (end 20.3702 10.792) (width 0.2) (layer "F.Cu") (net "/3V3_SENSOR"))
 (segment (start 28 9) (end 23.0308 9) (width 0.2) (layer "F.Cu") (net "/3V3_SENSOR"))
 (segment (start 20.3702 10.792) (end 19.9918 10.4136) (width 0.2) (layer "F.Cu") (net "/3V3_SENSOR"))
 (segment (start 37.045 8.73) (end 35 10.775) (width 0.2) (layer "F.Cu") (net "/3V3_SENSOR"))
 (segment (start 24.175 5.175) (end 24.175 5) (width 0.2) (layer "F.Cu") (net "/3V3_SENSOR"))
 (segment (start 18.6512 8.2299) (end 12.0801 8.2299) (width 0.2) (layer "F.Cu") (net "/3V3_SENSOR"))
 (segment (start 31.175 10.775) (end 29.775 10.775) (width 0.2) (layer "F.Cu") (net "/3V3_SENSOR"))
 (segment (start 11.84 8.47) (end 14.32 10.95) (width 0.2) (layer "F.Cu") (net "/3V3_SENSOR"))
 (segment (start 31.175 10.775) (end 31.175 12) (width 0.2) (layer "F.Cu") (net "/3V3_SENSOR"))
 (segment (start 28 9) (end 24.175 5.175) (width 0.2) (layer "F.Cu") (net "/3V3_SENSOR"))
 (segment (start 28.4307 12.95) (end 29 12.3807) (width 0.2) (layer "F.Cu") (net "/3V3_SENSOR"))
 (segment (start 24.0625 12.95) (end 28.4307 12.95) (width 0.2) (layer "F.Cu") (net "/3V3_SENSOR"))
 (segment (start 29 11.55) (end 29.775 10.775) (width 0.2) (layer "F.Cu") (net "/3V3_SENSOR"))
 (segment (start 35 10.775) (end 31.175 10.775) (width 0.2) (layer "F.Cu") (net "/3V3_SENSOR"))
 (segment (start 29 12.3807) (end 29 11.55) (width 0.2) (layer "F.Cu") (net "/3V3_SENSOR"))
 (segment (start 29.825 15.9625) (end 29.7875 16) (width 0.2) (layer "F.Cu") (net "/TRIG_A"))
 (segment (start 29.825 12) (end 29.825 15.9625) (width 0.2) (layer "F.Cu") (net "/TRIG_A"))
 (segment (start 20.1627 11.2007) (end 23.0083 11.2007) (width 0.2) (layer "F.Cu") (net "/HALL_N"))
 (segment (start 32.9317 12.1067) (end 32.825 12) (width 0.2) (layer "F.Cu") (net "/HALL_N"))
 (segment (start 19.175 10.213) (end 20.1627 11.2007) (width 0.2) (layer "F.Cu") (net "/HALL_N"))
 (segment (start 40 12.1067) (end 32.9317 12.1067) (width 0.2) (layer "F.Cu") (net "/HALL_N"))
 (segment (start 40 11.27) (end 40 12.1067) (width 0.2) (layer "F.Cu") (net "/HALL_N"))
 (segment (start 23.0083 13.3367) (end 23.0083 11.2007) (width 0.2) (layer "F.Cu") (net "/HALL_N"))
 (segment (start 28.9525 16.4793) (end 28.9525 15.4257) (width 0.2) (layer "F.Cu") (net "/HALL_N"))
 (segment (start 23.159 11.05) (end 24.0625 11.05) (width 0.2) (layer "F.Cu") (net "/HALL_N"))
 (segment (start 28.7493 15.2225) (end 24.8941 15.2225) (width 0.2) (layer "F.Cu") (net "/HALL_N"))
 (segment (start 19.175 10) (end 19.175 10.213) (width 0.2) (layer "F.Cu") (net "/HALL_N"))
 (segment (start 23.0083 11.2007) (end 23.159 11.05) (width 0.2) (layer "F.Cu") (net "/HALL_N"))
 (segment (start 24.8941 15.2225) (end 23.0083 13.3367) (width 0.2) (layer "F.Cu") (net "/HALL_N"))
 (segment (start 32.825 12) (end 32.825 14.2698) (width 0.2) (layer "F.Cu") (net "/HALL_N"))
 (segment (start 32.825 14.2698) (end 30.2829 16.8119) (width 0.2) (layer "F.Cu") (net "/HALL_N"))
 (segment (start 28.9525 15.4257) (end 28.7493 15.2225) (width 0.2) (layer "F.Cu") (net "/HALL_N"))
 (segment (start 29.2851 16.8119) (end 28.9525 16.4793) (width 0.2) (layer "F.Cu") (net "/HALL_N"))
 (segment (start 30.2829 16.8119) (end 29.2851 16.8119) (width 0.2) (layer "F.Cu") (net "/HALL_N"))
 (segment (start 28.175 12) (end 25.9375 12) (width 0.2) (layer "F.Cu") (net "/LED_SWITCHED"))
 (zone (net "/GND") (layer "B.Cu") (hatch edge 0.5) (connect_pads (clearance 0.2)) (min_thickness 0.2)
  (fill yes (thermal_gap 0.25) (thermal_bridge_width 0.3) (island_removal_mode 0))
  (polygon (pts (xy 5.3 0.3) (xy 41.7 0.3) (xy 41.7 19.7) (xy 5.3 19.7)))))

